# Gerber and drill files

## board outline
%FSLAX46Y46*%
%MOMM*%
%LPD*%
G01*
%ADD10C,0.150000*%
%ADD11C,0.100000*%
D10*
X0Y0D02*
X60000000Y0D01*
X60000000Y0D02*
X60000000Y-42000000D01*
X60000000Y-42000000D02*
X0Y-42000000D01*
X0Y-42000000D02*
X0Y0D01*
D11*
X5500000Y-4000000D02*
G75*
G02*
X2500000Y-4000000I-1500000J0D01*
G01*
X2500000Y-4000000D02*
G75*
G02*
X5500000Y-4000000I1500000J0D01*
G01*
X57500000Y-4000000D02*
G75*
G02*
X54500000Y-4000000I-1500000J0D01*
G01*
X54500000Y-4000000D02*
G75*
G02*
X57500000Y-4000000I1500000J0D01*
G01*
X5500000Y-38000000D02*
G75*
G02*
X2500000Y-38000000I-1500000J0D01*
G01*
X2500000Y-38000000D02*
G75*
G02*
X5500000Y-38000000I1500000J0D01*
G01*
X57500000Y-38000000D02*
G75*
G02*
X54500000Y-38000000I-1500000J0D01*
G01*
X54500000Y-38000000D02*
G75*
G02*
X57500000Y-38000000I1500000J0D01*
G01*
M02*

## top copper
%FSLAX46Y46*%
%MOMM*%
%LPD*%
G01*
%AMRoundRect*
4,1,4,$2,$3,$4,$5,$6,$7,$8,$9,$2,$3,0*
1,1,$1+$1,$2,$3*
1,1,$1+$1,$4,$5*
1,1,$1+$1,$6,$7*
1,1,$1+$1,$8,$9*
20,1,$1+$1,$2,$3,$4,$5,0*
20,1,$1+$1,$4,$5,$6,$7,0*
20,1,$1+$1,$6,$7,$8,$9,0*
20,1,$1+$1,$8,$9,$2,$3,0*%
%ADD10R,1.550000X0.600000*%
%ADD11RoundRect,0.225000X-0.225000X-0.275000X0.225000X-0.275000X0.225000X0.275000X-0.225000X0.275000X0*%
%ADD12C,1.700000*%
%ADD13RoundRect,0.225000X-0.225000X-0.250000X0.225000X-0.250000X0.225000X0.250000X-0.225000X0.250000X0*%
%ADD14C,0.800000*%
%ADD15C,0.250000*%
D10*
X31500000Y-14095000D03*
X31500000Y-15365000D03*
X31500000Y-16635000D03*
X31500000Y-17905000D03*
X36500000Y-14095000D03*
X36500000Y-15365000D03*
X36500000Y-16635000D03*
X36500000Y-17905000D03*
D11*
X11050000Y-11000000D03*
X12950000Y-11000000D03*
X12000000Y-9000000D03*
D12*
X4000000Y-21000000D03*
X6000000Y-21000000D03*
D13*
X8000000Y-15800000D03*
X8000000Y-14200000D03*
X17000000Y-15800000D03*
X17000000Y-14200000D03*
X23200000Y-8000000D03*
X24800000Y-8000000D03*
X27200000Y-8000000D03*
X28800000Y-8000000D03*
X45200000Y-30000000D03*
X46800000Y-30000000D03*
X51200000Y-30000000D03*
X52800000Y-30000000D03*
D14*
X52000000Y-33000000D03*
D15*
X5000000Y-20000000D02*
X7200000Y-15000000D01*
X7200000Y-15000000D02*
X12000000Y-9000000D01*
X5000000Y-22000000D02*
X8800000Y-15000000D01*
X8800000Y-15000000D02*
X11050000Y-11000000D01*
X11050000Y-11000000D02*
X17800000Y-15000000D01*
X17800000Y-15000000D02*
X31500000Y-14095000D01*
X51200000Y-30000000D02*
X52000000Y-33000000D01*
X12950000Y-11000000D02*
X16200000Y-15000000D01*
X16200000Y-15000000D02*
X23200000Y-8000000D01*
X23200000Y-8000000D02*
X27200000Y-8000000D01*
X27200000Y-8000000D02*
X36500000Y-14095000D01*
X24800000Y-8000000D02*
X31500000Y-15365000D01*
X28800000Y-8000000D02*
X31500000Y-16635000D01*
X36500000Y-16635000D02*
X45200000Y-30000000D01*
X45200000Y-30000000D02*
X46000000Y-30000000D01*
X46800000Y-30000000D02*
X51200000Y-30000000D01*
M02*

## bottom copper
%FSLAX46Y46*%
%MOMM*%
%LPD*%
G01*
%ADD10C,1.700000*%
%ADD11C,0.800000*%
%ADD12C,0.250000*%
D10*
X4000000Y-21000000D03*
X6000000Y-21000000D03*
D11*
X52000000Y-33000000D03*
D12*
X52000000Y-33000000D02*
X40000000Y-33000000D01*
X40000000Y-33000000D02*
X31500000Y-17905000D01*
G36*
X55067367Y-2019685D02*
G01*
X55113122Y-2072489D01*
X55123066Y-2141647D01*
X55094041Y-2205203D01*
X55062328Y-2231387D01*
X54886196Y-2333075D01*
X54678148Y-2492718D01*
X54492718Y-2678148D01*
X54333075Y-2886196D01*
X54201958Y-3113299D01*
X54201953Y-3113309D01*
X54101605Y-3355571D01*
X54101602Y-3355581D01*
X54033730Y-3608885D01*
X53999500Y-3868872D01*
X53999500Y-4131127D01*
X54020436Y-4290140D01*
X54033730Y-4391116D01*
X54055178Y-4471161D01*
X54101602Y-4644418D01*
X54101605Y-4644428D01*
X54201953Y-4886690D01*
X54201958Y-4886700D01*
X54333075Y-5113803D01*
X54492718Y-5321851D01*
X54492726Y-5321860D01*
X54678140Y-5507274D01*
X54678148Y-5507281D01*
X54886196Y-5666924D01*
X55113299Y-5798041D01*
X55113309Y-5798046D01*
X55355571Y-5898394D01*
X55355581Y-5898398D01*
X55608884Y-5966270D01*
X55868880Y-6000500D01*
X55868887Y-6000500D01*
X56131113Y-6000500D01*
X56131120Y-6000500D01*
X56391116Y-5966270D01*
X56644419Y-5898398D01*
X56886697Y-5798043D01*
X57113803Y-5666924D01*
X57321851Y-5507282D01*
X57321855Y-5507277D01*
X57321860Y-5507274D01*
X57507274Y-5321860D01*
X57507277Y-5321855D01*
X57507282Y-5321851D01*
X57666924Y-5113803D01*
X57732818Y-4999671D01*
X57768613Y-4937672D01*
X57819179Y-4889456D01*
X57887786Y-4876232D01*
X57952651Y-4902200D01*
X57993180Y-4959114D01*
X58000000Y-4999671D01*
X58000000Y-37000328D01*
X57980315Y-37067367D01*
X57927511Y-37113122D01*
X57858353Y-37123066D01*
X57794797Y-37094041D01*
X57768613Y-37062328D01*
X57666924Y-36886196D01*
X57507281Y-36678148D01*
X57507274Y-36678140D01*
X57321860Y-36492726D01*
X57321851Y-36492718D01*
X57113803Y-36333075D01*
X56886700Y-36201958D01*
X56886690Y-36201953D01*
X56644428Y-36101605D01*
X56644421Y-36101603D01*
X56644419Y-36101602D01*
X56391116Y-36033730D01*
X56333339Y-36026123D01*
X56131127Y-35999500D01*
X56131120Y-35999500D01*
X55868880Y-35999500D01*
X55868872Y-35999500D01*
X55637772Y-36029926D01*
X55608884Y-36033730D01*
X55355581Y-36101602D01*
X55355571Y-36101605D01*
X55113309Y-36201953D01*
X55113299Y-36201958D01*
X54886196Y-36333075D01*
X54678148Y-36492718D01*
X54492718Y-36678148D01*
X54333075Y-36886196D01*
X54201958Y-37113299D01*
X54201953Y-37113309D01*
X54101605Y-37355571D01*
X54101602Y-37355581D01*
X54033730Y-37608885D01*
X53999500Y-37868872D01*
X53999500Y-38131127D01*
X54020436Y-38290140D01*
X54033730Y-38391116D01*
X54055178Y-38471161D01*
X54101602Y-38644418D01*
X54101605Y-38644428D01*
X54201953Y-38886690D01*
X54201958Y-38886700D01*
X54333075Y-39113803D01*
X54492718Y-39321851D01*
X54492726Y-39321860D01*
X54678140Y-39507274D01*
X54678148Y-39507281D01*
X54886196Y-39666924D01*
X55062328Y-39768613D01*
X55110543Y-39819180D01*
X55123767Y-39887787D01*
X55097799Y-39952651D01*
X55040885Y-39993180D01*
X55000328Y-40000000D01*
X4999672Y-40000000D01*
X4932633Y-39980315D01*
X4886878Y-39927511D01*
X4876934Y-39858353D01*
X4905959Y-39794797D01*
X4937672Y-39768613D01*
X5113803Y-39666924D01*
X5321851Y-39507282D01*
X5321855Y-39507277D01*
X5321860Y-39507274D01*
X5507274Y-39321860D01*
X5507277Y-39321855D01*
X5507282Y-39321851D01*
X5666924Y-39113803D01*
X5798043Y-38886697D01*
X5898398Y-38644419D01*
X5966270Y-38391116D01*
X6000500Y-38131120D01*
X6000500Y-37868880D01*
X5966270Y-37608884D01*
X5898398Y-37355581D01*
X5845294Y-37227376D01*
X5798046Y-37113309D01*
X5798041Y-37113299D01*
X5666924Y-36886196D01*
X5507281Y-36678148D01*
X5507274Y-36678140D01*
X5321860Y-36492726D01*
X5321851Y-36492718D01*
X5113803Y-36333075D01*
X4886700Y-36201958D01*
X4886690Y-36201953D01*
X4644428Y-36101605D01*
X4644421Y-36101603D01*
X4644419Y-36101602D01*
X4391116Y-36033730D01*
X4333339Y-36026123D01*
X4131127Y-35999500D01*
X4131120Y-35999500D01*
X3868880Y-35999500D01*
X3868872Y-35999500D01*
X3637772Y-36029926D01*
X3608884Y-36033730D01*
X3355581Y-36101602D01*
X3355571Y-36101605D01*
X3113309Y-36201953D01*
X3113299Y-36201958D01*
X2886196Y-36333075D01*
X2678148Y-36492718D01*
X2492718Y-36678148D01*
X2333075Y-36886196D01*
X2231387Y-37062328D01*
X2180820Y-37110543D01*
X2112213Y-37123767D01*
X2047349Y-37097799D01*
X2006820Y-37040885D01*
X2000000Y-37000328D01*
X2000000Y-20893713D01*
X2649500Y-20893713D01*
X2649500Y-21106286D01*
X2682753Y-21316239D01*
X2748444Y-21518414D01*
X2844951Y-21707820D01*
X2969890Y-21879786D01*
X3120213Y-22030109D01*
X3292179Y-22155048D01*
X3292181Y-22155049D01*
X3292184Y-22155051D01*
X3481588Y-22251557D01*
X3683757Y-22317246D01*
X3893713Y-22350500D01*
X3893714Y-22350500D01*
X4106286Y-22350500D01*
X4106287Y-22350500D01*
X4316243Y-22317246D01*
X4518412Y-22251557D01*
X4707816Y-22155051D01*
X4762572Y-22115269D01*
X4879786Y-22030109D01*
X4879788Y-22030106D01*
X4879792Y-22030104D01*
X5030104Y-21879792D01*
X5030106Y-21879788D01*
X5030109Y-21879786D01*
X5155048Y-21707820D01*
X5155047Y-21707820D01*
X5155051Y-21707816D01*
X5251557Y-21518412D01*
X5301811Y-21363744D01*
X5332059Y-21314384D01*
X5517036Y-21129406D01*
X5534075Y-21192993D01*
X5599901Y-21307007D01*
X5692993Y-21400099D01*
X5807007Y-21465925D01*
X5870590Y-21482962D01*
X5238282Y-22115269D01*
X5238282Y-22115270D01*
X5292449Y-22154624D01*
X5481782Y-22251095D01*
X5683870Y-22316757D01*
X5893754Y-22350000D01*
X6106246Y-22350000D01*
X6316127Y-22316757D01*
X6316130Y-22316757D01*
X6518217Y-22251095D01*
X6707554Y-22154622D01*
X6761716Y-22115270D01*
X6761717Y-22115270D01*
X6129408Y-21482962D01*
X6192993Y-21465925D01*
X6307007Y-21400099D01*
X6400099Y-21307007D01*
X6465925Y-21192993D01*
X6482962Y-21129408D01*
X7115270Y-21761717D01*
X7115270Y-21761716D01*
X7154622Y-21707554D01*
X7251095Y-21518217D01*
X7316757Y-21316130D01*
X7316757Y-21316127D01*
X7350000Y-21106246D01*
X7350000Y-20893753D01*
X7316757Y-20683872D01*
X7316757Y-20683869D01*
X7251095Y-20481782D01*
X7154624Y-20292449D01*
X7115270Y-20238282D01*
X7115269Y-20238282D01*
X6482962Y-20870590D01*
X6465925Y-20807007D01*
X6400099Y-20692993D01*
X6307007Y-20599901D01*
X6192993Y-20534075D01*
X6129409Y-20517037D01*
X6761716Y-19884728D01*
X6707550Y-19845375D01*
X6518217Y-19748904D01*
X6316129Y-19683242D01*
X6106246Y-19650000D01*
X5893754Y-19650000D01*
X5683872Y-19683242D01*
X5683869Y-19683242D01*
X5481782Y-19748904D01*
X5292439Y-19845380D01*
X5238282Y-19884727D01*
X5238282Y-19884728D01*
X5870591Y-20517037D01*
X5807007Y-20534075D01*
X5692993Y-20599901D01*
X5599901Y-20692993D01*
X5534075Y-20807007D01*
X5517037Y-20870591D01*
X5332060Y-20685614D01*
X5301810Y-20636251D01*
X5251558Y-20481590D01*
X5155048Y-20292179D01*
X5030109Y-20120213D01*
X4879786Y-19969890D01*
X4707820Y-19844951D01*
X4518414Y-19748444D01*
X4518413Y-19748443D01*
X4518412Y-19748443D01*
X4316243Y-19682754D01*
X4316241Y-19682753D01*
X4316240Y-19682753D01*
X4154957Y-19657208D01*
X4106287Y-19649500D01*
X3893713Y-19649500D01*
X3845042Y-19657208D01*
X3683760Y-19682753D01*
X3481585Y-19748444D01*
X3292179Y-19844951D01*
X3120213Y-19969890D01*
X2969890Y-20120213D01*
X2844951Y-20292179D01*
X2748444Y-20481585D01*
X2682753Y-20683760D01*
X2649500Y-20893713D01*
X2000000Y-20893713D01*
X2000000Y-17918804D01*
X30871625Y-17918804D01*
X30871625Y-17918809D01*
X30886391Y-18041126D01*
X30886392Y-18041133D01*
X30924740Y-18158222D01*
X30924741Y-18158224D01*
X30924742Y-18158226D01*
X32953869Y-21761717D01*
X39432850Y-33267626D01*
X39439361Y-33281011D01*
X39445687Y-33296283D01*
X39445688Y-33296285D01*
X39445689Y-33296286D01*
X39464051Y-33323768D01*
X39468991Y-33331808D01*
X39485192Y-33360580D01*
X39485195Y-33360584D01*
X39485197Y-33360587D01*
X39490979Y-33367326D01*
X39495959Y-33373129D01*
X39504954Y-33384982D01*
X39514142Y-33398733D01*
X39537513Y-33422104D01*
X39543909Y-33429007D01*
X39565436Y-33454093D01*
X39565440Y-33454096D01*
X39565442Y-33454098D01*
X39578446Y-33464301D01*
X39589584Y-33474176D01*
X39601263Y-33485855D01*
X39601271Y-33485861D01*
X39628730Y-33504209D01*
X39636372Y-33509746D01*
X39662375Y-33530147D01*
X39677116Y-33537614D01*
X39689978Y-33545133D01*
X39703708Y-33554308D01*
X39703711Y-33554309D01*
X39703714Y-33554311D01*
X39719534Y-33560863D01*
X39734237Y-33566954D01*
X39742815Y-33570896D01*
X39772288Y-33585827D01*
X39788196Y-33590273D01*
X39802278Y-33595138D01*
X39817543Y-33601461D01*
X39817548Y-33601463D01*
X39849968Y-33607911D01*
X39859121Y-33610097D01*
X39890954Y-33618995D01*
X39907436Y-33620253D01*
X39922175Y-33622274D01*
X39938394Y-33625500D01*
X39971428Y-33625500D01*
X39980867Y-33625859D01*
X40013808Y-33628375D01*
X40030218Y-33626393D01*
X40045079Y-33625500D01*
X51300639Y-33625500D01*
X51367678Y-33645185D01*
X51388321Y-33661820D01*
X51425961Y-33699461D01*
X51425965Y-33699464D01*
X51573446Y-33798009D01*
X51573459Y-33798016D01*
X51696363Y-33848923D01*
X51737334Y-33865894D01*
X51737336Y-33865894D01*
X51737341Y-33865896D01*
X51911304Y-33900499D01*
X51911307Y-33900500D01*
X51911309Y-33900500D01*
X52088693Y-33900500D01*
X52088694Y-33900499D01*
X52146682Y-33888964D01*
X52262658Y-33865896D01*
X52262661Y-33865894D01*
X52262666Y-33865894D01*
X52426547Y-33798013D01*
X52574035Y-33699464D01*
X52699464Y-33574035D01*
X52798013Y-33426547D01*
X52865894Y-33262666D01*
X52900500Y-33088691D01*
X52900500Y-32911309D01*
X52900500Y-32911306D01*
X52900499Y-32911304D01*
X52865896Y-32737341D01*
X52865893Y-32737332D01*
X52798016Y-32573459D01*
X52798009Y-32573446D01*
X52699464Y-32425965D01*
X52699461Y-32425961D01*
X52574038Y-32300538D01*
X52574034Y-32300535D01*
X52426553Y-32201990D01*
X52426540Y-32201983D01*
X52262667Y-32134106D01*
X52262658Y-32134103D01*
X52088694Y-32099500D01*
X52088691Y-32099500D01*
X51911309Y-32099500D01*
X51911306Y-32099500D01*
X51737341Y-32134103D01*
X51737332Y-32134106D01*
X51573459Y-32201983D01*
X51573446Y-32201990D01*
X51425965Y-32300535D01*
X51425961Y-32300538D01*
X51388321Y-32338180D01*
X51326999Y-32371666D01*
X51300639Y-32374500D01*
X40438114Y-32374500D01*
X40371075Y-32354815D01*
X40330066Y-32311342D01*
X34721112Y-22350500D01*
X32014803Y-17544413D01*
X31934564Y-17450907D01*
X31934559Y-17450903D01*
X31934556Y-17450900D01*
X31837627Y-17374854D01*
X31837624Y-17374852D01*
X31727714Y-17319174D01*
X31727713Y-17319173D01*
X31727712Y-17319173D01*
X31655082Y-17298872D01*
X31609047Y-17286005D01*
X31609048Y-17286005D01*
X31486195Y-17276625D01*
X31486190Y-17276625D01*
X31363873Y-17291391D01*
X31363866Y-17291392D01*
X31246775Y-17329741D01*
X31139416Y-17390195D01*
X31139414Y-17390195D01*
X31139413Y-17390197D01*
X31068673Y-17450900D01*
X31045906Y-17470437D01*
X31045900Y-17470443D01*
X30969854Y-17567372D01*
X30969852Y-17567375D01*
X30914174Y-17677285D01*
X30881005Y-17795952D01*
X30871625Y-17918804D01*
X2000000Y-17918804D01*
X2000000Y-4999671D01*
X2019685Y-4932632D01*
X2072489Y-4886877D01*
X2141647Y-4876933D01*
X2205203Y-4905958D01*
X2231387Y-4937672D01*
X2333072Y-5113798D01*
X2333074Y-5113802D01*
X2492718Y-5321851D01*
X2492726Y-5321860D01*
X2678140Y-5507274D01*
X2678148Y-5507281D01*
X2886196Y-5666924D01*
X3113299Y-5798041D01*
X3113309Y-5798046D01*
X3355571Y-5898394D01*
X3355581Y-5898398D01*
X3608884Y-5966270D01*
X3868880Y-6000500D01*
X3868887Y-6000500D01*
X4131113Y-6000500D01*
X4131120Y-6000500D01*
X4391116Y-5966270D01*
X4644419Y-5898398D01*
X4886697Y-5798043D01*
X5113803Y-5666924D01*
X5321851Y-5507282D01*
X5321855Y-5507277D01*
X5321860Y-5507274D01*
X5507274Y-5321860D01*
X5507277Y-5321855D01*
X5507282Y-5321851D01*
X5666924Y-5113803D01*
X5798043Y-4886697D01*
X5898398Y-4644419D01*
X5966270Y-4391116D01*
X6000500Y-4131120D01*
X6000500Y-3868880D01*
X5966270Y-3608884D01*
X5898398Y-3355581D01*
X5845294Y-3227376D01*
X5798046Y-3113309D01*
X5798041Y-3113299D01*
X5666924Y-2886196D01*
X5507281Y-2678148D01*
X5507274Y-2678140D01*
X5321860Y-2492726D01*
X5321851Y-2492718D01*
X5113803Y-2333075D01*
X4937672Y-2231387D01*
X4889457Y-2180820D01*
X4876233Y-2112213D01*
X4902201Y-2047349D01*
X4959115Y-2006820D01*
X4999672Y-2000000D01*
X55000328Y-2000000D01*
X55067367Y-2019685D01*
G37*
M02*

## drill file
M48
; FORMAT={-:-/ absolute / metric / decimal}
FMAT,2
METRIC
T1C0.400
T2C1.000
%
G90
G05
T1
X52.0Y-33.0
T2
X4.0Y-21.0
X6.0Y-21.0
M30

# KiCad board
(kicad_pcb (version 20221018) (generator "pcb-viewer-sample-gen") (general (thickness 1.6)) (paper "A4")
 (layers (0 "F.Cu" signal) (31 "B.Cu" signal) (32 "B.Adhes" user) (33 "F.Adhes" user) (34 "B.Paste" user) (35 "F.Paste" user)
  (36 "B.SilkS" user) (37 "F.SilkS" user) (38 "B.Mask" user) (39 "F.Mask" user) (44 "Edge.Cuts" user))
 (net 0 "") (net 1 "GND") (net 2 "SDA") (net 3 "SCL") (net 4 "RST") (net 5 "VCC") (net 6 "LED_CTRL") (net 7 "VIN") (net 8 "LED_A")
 (gr_line (start 0 0) (end 60 0) (layer "Edge.Cuts") (width 0.15))
 (gr_line (start 60 0) (end 60 42) (layer "Edge.Cuts") (width 0.15))
 (gr_line (start 60 42) (end 0 42) (layer "Edge.Cuts") (width 0.15))
 (gr_line (start 0 42) (end 0 0) (layer "Edge.Cuts") (width 0.15))
 (gr_circle (center 4 4) (end 5.5 4) (layer "Edge.Cuts") (width 0.1))
 (gr_circle (center 56 4) (end 57.5 4) (layer "Edge.Cuts") (width 0.1))
 (gr_circle (center 4 38) (end 5.5 38) (layer "Edge.Cuts") (width 0.1))
 (gr_circle (center 56 38) (end 57.5 38) (layer "Edge.Cuts") (width 0.1))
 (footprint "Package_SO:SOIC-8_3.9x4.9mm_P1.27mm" (layer "F.Cu") (at 34 16)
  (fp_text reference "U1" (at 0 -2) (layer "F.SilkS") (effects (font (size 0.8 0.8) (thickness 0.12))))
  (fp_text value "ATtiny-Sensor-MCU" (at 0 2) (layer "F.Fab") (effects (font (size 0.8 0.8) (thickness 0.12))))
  (pad "1" smd rect (at -2.5 -1.905) (size 1.55 0.6) (layers "F.Cu" "F.Paste" "F.Mask") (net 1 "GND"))
  (pad "2" smd rect (at -2.5 -0.635) (size 1.55 0.6) (layers "F.Cu" "F.Paste" "F.Mask") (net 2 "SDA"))
  (pad "3" smd rect (at -2.5 0.635) (size 1.55 0.6) (layers "F.Cu" "F.Paste" "F.Mask") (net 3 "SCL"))
  (pad "4" smd rect (at -2.5 1.905) (size 1.55 0.6) (layers "F.Cu" "F.Paste" "F.Mask") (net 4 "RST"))
  (pad "8" smd rect (at 2.5 -1.905) (size 1.55 0.6) (layers "F.Cu" "F.Paste" "F.Mask") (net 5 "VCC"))
  (pad "7" smd rect (at 2.5 -0.635) (size 1.55 0.6) (layers "F.Cu" "F.Paste" "F.Mask"))
  (pad "6" smd rect (at 2.5 0.635) (size 1.55 0.6) (layers "F.Cu" "F.Paste" "F.Mask"))
  (pad "5" smd rect (at 2.5 1.905) (size 1.55 0.6) (layers "F.Cu" "F.Paste" "F.Mask") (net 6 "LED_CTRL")))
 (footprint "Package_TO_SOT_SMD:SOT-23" (layer "F.Cu") (at 12 10)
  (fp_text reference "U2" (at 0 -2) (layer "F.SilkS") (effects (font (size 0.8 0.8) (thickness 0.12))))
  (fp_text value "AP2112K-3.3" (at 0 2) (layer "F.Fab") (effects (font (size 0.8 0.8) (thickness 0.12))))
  (pad "1" smd roundrect (at -0.95 1) (size 0.9 1) (layers "F.Cu" "F.Paste" "F.Mask") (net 1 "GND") (roundrect_rratio 0.25))
  (pad "2" smd roundrect (at 0.95 1) (size 0.9 1) (layers "F.Cu" "F.Paste" "F.Mask") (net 5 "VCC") (roundrect_rratio 0.25))
  (pad "3" smd roundrect (at 0 -1) (size 0.9 1) (layers "F.Cu" "F.Paste" "F.Mask") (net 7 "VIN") (roundrect_rratio 0.25)))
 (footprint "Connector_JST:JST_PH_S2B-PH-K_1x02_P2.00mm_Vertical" (layer "F.Cu") (at 5 21 90)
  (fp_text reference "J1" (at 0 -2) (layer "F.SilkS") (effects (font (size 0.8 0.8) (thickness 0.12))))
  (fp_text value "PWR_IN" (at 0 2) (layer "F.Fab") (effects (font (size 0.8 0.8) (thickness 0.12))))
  (pad "1" thru_hole circle (at 0 -1) (size 1.7 1.7) (drill 1) (layers "*.Cu" "*.Mask") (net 7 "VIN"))
  (pad "2" thru_hole circle (at 0 1) (size 1.7 1.7) (drill 1) (layers "*.Cu" "*.Mask") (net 1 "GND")))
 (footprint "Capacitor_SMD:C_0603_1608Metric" (layer "F.Cu") (at 8 15 90)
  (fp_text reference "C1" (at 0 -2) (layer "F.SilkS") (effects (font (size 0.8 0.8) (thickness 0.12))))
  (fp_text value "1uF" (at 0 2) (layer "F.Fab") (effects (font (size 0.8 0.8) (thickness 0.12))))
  (pad "1" smd roundrect (at -0.8 0) (size 0.9 0.95) (layers "F.Cu" "F.Paste" "F.Mask") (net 7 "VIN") (roundrect_rratio 0.25))
  (pad "2" smd roundrect (at 0.8 0) (size 0.9 0.95) (layers "F.Cu" "F.Paste" "F.Mask") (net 1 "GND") (roundrect_rratio 0.25)))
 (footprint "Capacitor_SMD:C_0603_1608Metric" (layer "F.Cu") (at 17 15 90)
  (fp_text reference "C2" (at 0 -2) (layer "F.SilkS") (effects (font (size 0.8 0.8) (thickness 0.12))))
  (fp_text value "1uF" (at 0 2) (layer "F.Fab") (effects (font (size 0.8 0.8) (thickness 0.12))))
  (pad "1" smd roundrect (at -0.8 0) (size 0.9 0.95) (layers "F.Cu" "F.Paste" "F.Mask") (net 5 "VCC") (roundrect_rratio 0.25))
  (pad "2" smd roundrect (at 0.8 0) (size 0.9 0.95) (layers "F.Cu" "F.Paste" "F.Mask") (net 1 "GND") (roundrect_rratio 0.25)))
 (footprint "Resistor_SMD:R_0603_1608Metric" (layer "F.Cu") (at 24 8)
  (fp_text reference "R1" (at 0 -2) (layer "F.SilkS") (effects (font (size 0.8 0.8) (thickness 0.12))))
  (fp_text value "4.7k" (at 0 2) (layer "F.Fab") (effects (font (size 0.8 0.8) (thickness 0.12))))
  (pad "1" smd roundrect (at -0.8 0) (size 0.9 0.95) (layers "F.Cu" "F.Paste" "F.Mask") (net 5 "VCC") (roundrect_rratio 0.25))
  (pad "2" smd roundrect (at 0.8 0) (size 0.9 0.95) (layers "F.Cu" "F.Paste" "F.Mask") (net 2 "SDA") (roundrect_rratio 0.25)))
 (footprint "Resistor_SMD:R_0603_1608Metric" (layer "F.Cu") (at 28 8)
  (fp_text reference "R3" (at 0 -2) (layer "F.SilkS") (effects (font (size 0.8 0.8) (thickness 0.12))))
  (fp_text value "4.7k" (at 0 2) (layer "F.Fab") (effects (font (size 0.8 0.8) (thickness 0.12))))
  (pad "1" smd roundrect (at -0.8 0) (size 0.9 0.95) (layers "F.Cu" "F.Paste" "F.Mask") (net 5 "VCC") (roundrect_rratio 0.25))
  (pad "2" smd roundrect (at 0.8 0) (size 0.9 0.95) (layers "F.Cu" "F.Paste" "F.Mask") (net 3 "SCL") (roundrect_rratio 0.25)))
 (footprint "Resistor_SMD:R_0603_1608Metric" (layer "F.Cu") (at 46 30)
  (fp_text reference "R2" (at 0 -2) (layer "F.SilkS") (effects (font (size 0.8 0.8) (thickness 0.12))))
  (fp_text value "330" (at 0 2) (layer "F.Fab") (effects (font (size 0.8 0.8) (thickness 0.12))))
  (pad "1" smd roundrect (at -0.8 0) (size 0.9 0.95) (layers "F.Cu" "F.Paste" "F.Mask") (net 6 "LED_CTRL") (roundrect_rratio 0.25))
  (pad "2" smd roundrect (at 0.8 0) (size 0.9 0.95) (layers "F.Cu" "F.Paste" "F.Mask") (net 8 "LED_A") (roundrect_rratio 0.25)))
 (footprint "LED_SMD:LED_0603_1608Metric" (layer "F.Cu") (at 52 30)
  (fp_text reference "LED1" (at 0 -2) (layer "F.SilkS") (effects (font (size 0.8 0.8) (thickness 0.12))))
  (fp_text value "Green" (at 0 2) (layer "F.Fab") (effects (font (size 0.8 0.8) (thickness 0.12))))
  (pad "1" smd roundrect (at -0.8 0) (size 0.9 0.95) (layers "F.Cu" "F.Paste" "F.Mask") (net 8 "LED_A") (roundrect_rratio 0.25))
  (pad "2" smd roundrect (at 0.8 0) (size 0.9 0.95) (layers "F.Cu" "F.Paste" "F.Mask") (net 1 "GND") (roundrect_rratio 0.25)))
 (segment (start 5 20) (end 7.2 15) (width 0.25) (layer "F.Cu") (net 7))
 (segment (start 7.2 15) (end 12 9) (width 0.25) (layer "F.Cu") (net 7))
 (segment (start 5 22) (end 8.8 15) (width 0.25) (layer "F.Cu") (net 1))
 (segment (start 8.8 15) (end 11.05 11) (width 0.25) (layer "F.Cu") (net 1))
 (segment (start 11.05 11) (end 17.8 15) (width 0.25) (layer "F.Cu") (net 1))
 (segment (start 17.8 15) (end 31.5 14.095) (width 0.25) (layer "F.Cu") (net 1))
 (segment (start 51.2 30) (end 52 33) (width 0.25) (layer "F.Cu") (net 1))
 (via (at 52 33) (size 0.8) (drill 0.4) (layers "F.Cu" "B.Cu") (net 1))
 (segment (start 52 33) (end 40 33) (width 0.25) (layer "B.Cu") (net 1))
 (segment (start 40 33) (end 31.5 17.905) (width 0.25) (layer "B.Cu") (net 1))
 (segment (start 12.95 11) (end 16.2 15) (width 0.25) (layer "F.Cu") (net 5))
 (segment (start 16.2 15) (end 23.2 8) (width 0.25) (layer "F.Cu") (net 5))
 (segment (start 23.2 8) (end 27.2 8) (width 0.25) (layer "F.Cu") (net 5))
 (segment (start 27.2 8) (end 36.5 14.095) (width 0.25) (layer "F.Cu") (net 5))
 (segment (start 24.8 8) (end 31.5 15.365) (width 0.25) (layer "F.Cu") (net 2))
 (segment (start 28.8 8) (end 31.5 16.635) (width 0.25) (layer "F.Cu") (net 3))
 (segment (start 36.5 16.635) (end 45.2 30) (width 0.25) (layer "F.Cu") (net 6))
 (segment (start 45.2 30) (end 46 30) (width 0.25) (layer "F.Cu") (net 6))
 (segment (start 46.8 30) (end 51.2 30) (width 0.25) (layer "F.Cu") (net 8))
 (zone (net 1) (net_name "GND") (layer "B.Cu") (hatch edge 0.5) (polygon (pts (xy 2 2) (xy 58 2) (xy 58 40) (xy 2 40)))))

